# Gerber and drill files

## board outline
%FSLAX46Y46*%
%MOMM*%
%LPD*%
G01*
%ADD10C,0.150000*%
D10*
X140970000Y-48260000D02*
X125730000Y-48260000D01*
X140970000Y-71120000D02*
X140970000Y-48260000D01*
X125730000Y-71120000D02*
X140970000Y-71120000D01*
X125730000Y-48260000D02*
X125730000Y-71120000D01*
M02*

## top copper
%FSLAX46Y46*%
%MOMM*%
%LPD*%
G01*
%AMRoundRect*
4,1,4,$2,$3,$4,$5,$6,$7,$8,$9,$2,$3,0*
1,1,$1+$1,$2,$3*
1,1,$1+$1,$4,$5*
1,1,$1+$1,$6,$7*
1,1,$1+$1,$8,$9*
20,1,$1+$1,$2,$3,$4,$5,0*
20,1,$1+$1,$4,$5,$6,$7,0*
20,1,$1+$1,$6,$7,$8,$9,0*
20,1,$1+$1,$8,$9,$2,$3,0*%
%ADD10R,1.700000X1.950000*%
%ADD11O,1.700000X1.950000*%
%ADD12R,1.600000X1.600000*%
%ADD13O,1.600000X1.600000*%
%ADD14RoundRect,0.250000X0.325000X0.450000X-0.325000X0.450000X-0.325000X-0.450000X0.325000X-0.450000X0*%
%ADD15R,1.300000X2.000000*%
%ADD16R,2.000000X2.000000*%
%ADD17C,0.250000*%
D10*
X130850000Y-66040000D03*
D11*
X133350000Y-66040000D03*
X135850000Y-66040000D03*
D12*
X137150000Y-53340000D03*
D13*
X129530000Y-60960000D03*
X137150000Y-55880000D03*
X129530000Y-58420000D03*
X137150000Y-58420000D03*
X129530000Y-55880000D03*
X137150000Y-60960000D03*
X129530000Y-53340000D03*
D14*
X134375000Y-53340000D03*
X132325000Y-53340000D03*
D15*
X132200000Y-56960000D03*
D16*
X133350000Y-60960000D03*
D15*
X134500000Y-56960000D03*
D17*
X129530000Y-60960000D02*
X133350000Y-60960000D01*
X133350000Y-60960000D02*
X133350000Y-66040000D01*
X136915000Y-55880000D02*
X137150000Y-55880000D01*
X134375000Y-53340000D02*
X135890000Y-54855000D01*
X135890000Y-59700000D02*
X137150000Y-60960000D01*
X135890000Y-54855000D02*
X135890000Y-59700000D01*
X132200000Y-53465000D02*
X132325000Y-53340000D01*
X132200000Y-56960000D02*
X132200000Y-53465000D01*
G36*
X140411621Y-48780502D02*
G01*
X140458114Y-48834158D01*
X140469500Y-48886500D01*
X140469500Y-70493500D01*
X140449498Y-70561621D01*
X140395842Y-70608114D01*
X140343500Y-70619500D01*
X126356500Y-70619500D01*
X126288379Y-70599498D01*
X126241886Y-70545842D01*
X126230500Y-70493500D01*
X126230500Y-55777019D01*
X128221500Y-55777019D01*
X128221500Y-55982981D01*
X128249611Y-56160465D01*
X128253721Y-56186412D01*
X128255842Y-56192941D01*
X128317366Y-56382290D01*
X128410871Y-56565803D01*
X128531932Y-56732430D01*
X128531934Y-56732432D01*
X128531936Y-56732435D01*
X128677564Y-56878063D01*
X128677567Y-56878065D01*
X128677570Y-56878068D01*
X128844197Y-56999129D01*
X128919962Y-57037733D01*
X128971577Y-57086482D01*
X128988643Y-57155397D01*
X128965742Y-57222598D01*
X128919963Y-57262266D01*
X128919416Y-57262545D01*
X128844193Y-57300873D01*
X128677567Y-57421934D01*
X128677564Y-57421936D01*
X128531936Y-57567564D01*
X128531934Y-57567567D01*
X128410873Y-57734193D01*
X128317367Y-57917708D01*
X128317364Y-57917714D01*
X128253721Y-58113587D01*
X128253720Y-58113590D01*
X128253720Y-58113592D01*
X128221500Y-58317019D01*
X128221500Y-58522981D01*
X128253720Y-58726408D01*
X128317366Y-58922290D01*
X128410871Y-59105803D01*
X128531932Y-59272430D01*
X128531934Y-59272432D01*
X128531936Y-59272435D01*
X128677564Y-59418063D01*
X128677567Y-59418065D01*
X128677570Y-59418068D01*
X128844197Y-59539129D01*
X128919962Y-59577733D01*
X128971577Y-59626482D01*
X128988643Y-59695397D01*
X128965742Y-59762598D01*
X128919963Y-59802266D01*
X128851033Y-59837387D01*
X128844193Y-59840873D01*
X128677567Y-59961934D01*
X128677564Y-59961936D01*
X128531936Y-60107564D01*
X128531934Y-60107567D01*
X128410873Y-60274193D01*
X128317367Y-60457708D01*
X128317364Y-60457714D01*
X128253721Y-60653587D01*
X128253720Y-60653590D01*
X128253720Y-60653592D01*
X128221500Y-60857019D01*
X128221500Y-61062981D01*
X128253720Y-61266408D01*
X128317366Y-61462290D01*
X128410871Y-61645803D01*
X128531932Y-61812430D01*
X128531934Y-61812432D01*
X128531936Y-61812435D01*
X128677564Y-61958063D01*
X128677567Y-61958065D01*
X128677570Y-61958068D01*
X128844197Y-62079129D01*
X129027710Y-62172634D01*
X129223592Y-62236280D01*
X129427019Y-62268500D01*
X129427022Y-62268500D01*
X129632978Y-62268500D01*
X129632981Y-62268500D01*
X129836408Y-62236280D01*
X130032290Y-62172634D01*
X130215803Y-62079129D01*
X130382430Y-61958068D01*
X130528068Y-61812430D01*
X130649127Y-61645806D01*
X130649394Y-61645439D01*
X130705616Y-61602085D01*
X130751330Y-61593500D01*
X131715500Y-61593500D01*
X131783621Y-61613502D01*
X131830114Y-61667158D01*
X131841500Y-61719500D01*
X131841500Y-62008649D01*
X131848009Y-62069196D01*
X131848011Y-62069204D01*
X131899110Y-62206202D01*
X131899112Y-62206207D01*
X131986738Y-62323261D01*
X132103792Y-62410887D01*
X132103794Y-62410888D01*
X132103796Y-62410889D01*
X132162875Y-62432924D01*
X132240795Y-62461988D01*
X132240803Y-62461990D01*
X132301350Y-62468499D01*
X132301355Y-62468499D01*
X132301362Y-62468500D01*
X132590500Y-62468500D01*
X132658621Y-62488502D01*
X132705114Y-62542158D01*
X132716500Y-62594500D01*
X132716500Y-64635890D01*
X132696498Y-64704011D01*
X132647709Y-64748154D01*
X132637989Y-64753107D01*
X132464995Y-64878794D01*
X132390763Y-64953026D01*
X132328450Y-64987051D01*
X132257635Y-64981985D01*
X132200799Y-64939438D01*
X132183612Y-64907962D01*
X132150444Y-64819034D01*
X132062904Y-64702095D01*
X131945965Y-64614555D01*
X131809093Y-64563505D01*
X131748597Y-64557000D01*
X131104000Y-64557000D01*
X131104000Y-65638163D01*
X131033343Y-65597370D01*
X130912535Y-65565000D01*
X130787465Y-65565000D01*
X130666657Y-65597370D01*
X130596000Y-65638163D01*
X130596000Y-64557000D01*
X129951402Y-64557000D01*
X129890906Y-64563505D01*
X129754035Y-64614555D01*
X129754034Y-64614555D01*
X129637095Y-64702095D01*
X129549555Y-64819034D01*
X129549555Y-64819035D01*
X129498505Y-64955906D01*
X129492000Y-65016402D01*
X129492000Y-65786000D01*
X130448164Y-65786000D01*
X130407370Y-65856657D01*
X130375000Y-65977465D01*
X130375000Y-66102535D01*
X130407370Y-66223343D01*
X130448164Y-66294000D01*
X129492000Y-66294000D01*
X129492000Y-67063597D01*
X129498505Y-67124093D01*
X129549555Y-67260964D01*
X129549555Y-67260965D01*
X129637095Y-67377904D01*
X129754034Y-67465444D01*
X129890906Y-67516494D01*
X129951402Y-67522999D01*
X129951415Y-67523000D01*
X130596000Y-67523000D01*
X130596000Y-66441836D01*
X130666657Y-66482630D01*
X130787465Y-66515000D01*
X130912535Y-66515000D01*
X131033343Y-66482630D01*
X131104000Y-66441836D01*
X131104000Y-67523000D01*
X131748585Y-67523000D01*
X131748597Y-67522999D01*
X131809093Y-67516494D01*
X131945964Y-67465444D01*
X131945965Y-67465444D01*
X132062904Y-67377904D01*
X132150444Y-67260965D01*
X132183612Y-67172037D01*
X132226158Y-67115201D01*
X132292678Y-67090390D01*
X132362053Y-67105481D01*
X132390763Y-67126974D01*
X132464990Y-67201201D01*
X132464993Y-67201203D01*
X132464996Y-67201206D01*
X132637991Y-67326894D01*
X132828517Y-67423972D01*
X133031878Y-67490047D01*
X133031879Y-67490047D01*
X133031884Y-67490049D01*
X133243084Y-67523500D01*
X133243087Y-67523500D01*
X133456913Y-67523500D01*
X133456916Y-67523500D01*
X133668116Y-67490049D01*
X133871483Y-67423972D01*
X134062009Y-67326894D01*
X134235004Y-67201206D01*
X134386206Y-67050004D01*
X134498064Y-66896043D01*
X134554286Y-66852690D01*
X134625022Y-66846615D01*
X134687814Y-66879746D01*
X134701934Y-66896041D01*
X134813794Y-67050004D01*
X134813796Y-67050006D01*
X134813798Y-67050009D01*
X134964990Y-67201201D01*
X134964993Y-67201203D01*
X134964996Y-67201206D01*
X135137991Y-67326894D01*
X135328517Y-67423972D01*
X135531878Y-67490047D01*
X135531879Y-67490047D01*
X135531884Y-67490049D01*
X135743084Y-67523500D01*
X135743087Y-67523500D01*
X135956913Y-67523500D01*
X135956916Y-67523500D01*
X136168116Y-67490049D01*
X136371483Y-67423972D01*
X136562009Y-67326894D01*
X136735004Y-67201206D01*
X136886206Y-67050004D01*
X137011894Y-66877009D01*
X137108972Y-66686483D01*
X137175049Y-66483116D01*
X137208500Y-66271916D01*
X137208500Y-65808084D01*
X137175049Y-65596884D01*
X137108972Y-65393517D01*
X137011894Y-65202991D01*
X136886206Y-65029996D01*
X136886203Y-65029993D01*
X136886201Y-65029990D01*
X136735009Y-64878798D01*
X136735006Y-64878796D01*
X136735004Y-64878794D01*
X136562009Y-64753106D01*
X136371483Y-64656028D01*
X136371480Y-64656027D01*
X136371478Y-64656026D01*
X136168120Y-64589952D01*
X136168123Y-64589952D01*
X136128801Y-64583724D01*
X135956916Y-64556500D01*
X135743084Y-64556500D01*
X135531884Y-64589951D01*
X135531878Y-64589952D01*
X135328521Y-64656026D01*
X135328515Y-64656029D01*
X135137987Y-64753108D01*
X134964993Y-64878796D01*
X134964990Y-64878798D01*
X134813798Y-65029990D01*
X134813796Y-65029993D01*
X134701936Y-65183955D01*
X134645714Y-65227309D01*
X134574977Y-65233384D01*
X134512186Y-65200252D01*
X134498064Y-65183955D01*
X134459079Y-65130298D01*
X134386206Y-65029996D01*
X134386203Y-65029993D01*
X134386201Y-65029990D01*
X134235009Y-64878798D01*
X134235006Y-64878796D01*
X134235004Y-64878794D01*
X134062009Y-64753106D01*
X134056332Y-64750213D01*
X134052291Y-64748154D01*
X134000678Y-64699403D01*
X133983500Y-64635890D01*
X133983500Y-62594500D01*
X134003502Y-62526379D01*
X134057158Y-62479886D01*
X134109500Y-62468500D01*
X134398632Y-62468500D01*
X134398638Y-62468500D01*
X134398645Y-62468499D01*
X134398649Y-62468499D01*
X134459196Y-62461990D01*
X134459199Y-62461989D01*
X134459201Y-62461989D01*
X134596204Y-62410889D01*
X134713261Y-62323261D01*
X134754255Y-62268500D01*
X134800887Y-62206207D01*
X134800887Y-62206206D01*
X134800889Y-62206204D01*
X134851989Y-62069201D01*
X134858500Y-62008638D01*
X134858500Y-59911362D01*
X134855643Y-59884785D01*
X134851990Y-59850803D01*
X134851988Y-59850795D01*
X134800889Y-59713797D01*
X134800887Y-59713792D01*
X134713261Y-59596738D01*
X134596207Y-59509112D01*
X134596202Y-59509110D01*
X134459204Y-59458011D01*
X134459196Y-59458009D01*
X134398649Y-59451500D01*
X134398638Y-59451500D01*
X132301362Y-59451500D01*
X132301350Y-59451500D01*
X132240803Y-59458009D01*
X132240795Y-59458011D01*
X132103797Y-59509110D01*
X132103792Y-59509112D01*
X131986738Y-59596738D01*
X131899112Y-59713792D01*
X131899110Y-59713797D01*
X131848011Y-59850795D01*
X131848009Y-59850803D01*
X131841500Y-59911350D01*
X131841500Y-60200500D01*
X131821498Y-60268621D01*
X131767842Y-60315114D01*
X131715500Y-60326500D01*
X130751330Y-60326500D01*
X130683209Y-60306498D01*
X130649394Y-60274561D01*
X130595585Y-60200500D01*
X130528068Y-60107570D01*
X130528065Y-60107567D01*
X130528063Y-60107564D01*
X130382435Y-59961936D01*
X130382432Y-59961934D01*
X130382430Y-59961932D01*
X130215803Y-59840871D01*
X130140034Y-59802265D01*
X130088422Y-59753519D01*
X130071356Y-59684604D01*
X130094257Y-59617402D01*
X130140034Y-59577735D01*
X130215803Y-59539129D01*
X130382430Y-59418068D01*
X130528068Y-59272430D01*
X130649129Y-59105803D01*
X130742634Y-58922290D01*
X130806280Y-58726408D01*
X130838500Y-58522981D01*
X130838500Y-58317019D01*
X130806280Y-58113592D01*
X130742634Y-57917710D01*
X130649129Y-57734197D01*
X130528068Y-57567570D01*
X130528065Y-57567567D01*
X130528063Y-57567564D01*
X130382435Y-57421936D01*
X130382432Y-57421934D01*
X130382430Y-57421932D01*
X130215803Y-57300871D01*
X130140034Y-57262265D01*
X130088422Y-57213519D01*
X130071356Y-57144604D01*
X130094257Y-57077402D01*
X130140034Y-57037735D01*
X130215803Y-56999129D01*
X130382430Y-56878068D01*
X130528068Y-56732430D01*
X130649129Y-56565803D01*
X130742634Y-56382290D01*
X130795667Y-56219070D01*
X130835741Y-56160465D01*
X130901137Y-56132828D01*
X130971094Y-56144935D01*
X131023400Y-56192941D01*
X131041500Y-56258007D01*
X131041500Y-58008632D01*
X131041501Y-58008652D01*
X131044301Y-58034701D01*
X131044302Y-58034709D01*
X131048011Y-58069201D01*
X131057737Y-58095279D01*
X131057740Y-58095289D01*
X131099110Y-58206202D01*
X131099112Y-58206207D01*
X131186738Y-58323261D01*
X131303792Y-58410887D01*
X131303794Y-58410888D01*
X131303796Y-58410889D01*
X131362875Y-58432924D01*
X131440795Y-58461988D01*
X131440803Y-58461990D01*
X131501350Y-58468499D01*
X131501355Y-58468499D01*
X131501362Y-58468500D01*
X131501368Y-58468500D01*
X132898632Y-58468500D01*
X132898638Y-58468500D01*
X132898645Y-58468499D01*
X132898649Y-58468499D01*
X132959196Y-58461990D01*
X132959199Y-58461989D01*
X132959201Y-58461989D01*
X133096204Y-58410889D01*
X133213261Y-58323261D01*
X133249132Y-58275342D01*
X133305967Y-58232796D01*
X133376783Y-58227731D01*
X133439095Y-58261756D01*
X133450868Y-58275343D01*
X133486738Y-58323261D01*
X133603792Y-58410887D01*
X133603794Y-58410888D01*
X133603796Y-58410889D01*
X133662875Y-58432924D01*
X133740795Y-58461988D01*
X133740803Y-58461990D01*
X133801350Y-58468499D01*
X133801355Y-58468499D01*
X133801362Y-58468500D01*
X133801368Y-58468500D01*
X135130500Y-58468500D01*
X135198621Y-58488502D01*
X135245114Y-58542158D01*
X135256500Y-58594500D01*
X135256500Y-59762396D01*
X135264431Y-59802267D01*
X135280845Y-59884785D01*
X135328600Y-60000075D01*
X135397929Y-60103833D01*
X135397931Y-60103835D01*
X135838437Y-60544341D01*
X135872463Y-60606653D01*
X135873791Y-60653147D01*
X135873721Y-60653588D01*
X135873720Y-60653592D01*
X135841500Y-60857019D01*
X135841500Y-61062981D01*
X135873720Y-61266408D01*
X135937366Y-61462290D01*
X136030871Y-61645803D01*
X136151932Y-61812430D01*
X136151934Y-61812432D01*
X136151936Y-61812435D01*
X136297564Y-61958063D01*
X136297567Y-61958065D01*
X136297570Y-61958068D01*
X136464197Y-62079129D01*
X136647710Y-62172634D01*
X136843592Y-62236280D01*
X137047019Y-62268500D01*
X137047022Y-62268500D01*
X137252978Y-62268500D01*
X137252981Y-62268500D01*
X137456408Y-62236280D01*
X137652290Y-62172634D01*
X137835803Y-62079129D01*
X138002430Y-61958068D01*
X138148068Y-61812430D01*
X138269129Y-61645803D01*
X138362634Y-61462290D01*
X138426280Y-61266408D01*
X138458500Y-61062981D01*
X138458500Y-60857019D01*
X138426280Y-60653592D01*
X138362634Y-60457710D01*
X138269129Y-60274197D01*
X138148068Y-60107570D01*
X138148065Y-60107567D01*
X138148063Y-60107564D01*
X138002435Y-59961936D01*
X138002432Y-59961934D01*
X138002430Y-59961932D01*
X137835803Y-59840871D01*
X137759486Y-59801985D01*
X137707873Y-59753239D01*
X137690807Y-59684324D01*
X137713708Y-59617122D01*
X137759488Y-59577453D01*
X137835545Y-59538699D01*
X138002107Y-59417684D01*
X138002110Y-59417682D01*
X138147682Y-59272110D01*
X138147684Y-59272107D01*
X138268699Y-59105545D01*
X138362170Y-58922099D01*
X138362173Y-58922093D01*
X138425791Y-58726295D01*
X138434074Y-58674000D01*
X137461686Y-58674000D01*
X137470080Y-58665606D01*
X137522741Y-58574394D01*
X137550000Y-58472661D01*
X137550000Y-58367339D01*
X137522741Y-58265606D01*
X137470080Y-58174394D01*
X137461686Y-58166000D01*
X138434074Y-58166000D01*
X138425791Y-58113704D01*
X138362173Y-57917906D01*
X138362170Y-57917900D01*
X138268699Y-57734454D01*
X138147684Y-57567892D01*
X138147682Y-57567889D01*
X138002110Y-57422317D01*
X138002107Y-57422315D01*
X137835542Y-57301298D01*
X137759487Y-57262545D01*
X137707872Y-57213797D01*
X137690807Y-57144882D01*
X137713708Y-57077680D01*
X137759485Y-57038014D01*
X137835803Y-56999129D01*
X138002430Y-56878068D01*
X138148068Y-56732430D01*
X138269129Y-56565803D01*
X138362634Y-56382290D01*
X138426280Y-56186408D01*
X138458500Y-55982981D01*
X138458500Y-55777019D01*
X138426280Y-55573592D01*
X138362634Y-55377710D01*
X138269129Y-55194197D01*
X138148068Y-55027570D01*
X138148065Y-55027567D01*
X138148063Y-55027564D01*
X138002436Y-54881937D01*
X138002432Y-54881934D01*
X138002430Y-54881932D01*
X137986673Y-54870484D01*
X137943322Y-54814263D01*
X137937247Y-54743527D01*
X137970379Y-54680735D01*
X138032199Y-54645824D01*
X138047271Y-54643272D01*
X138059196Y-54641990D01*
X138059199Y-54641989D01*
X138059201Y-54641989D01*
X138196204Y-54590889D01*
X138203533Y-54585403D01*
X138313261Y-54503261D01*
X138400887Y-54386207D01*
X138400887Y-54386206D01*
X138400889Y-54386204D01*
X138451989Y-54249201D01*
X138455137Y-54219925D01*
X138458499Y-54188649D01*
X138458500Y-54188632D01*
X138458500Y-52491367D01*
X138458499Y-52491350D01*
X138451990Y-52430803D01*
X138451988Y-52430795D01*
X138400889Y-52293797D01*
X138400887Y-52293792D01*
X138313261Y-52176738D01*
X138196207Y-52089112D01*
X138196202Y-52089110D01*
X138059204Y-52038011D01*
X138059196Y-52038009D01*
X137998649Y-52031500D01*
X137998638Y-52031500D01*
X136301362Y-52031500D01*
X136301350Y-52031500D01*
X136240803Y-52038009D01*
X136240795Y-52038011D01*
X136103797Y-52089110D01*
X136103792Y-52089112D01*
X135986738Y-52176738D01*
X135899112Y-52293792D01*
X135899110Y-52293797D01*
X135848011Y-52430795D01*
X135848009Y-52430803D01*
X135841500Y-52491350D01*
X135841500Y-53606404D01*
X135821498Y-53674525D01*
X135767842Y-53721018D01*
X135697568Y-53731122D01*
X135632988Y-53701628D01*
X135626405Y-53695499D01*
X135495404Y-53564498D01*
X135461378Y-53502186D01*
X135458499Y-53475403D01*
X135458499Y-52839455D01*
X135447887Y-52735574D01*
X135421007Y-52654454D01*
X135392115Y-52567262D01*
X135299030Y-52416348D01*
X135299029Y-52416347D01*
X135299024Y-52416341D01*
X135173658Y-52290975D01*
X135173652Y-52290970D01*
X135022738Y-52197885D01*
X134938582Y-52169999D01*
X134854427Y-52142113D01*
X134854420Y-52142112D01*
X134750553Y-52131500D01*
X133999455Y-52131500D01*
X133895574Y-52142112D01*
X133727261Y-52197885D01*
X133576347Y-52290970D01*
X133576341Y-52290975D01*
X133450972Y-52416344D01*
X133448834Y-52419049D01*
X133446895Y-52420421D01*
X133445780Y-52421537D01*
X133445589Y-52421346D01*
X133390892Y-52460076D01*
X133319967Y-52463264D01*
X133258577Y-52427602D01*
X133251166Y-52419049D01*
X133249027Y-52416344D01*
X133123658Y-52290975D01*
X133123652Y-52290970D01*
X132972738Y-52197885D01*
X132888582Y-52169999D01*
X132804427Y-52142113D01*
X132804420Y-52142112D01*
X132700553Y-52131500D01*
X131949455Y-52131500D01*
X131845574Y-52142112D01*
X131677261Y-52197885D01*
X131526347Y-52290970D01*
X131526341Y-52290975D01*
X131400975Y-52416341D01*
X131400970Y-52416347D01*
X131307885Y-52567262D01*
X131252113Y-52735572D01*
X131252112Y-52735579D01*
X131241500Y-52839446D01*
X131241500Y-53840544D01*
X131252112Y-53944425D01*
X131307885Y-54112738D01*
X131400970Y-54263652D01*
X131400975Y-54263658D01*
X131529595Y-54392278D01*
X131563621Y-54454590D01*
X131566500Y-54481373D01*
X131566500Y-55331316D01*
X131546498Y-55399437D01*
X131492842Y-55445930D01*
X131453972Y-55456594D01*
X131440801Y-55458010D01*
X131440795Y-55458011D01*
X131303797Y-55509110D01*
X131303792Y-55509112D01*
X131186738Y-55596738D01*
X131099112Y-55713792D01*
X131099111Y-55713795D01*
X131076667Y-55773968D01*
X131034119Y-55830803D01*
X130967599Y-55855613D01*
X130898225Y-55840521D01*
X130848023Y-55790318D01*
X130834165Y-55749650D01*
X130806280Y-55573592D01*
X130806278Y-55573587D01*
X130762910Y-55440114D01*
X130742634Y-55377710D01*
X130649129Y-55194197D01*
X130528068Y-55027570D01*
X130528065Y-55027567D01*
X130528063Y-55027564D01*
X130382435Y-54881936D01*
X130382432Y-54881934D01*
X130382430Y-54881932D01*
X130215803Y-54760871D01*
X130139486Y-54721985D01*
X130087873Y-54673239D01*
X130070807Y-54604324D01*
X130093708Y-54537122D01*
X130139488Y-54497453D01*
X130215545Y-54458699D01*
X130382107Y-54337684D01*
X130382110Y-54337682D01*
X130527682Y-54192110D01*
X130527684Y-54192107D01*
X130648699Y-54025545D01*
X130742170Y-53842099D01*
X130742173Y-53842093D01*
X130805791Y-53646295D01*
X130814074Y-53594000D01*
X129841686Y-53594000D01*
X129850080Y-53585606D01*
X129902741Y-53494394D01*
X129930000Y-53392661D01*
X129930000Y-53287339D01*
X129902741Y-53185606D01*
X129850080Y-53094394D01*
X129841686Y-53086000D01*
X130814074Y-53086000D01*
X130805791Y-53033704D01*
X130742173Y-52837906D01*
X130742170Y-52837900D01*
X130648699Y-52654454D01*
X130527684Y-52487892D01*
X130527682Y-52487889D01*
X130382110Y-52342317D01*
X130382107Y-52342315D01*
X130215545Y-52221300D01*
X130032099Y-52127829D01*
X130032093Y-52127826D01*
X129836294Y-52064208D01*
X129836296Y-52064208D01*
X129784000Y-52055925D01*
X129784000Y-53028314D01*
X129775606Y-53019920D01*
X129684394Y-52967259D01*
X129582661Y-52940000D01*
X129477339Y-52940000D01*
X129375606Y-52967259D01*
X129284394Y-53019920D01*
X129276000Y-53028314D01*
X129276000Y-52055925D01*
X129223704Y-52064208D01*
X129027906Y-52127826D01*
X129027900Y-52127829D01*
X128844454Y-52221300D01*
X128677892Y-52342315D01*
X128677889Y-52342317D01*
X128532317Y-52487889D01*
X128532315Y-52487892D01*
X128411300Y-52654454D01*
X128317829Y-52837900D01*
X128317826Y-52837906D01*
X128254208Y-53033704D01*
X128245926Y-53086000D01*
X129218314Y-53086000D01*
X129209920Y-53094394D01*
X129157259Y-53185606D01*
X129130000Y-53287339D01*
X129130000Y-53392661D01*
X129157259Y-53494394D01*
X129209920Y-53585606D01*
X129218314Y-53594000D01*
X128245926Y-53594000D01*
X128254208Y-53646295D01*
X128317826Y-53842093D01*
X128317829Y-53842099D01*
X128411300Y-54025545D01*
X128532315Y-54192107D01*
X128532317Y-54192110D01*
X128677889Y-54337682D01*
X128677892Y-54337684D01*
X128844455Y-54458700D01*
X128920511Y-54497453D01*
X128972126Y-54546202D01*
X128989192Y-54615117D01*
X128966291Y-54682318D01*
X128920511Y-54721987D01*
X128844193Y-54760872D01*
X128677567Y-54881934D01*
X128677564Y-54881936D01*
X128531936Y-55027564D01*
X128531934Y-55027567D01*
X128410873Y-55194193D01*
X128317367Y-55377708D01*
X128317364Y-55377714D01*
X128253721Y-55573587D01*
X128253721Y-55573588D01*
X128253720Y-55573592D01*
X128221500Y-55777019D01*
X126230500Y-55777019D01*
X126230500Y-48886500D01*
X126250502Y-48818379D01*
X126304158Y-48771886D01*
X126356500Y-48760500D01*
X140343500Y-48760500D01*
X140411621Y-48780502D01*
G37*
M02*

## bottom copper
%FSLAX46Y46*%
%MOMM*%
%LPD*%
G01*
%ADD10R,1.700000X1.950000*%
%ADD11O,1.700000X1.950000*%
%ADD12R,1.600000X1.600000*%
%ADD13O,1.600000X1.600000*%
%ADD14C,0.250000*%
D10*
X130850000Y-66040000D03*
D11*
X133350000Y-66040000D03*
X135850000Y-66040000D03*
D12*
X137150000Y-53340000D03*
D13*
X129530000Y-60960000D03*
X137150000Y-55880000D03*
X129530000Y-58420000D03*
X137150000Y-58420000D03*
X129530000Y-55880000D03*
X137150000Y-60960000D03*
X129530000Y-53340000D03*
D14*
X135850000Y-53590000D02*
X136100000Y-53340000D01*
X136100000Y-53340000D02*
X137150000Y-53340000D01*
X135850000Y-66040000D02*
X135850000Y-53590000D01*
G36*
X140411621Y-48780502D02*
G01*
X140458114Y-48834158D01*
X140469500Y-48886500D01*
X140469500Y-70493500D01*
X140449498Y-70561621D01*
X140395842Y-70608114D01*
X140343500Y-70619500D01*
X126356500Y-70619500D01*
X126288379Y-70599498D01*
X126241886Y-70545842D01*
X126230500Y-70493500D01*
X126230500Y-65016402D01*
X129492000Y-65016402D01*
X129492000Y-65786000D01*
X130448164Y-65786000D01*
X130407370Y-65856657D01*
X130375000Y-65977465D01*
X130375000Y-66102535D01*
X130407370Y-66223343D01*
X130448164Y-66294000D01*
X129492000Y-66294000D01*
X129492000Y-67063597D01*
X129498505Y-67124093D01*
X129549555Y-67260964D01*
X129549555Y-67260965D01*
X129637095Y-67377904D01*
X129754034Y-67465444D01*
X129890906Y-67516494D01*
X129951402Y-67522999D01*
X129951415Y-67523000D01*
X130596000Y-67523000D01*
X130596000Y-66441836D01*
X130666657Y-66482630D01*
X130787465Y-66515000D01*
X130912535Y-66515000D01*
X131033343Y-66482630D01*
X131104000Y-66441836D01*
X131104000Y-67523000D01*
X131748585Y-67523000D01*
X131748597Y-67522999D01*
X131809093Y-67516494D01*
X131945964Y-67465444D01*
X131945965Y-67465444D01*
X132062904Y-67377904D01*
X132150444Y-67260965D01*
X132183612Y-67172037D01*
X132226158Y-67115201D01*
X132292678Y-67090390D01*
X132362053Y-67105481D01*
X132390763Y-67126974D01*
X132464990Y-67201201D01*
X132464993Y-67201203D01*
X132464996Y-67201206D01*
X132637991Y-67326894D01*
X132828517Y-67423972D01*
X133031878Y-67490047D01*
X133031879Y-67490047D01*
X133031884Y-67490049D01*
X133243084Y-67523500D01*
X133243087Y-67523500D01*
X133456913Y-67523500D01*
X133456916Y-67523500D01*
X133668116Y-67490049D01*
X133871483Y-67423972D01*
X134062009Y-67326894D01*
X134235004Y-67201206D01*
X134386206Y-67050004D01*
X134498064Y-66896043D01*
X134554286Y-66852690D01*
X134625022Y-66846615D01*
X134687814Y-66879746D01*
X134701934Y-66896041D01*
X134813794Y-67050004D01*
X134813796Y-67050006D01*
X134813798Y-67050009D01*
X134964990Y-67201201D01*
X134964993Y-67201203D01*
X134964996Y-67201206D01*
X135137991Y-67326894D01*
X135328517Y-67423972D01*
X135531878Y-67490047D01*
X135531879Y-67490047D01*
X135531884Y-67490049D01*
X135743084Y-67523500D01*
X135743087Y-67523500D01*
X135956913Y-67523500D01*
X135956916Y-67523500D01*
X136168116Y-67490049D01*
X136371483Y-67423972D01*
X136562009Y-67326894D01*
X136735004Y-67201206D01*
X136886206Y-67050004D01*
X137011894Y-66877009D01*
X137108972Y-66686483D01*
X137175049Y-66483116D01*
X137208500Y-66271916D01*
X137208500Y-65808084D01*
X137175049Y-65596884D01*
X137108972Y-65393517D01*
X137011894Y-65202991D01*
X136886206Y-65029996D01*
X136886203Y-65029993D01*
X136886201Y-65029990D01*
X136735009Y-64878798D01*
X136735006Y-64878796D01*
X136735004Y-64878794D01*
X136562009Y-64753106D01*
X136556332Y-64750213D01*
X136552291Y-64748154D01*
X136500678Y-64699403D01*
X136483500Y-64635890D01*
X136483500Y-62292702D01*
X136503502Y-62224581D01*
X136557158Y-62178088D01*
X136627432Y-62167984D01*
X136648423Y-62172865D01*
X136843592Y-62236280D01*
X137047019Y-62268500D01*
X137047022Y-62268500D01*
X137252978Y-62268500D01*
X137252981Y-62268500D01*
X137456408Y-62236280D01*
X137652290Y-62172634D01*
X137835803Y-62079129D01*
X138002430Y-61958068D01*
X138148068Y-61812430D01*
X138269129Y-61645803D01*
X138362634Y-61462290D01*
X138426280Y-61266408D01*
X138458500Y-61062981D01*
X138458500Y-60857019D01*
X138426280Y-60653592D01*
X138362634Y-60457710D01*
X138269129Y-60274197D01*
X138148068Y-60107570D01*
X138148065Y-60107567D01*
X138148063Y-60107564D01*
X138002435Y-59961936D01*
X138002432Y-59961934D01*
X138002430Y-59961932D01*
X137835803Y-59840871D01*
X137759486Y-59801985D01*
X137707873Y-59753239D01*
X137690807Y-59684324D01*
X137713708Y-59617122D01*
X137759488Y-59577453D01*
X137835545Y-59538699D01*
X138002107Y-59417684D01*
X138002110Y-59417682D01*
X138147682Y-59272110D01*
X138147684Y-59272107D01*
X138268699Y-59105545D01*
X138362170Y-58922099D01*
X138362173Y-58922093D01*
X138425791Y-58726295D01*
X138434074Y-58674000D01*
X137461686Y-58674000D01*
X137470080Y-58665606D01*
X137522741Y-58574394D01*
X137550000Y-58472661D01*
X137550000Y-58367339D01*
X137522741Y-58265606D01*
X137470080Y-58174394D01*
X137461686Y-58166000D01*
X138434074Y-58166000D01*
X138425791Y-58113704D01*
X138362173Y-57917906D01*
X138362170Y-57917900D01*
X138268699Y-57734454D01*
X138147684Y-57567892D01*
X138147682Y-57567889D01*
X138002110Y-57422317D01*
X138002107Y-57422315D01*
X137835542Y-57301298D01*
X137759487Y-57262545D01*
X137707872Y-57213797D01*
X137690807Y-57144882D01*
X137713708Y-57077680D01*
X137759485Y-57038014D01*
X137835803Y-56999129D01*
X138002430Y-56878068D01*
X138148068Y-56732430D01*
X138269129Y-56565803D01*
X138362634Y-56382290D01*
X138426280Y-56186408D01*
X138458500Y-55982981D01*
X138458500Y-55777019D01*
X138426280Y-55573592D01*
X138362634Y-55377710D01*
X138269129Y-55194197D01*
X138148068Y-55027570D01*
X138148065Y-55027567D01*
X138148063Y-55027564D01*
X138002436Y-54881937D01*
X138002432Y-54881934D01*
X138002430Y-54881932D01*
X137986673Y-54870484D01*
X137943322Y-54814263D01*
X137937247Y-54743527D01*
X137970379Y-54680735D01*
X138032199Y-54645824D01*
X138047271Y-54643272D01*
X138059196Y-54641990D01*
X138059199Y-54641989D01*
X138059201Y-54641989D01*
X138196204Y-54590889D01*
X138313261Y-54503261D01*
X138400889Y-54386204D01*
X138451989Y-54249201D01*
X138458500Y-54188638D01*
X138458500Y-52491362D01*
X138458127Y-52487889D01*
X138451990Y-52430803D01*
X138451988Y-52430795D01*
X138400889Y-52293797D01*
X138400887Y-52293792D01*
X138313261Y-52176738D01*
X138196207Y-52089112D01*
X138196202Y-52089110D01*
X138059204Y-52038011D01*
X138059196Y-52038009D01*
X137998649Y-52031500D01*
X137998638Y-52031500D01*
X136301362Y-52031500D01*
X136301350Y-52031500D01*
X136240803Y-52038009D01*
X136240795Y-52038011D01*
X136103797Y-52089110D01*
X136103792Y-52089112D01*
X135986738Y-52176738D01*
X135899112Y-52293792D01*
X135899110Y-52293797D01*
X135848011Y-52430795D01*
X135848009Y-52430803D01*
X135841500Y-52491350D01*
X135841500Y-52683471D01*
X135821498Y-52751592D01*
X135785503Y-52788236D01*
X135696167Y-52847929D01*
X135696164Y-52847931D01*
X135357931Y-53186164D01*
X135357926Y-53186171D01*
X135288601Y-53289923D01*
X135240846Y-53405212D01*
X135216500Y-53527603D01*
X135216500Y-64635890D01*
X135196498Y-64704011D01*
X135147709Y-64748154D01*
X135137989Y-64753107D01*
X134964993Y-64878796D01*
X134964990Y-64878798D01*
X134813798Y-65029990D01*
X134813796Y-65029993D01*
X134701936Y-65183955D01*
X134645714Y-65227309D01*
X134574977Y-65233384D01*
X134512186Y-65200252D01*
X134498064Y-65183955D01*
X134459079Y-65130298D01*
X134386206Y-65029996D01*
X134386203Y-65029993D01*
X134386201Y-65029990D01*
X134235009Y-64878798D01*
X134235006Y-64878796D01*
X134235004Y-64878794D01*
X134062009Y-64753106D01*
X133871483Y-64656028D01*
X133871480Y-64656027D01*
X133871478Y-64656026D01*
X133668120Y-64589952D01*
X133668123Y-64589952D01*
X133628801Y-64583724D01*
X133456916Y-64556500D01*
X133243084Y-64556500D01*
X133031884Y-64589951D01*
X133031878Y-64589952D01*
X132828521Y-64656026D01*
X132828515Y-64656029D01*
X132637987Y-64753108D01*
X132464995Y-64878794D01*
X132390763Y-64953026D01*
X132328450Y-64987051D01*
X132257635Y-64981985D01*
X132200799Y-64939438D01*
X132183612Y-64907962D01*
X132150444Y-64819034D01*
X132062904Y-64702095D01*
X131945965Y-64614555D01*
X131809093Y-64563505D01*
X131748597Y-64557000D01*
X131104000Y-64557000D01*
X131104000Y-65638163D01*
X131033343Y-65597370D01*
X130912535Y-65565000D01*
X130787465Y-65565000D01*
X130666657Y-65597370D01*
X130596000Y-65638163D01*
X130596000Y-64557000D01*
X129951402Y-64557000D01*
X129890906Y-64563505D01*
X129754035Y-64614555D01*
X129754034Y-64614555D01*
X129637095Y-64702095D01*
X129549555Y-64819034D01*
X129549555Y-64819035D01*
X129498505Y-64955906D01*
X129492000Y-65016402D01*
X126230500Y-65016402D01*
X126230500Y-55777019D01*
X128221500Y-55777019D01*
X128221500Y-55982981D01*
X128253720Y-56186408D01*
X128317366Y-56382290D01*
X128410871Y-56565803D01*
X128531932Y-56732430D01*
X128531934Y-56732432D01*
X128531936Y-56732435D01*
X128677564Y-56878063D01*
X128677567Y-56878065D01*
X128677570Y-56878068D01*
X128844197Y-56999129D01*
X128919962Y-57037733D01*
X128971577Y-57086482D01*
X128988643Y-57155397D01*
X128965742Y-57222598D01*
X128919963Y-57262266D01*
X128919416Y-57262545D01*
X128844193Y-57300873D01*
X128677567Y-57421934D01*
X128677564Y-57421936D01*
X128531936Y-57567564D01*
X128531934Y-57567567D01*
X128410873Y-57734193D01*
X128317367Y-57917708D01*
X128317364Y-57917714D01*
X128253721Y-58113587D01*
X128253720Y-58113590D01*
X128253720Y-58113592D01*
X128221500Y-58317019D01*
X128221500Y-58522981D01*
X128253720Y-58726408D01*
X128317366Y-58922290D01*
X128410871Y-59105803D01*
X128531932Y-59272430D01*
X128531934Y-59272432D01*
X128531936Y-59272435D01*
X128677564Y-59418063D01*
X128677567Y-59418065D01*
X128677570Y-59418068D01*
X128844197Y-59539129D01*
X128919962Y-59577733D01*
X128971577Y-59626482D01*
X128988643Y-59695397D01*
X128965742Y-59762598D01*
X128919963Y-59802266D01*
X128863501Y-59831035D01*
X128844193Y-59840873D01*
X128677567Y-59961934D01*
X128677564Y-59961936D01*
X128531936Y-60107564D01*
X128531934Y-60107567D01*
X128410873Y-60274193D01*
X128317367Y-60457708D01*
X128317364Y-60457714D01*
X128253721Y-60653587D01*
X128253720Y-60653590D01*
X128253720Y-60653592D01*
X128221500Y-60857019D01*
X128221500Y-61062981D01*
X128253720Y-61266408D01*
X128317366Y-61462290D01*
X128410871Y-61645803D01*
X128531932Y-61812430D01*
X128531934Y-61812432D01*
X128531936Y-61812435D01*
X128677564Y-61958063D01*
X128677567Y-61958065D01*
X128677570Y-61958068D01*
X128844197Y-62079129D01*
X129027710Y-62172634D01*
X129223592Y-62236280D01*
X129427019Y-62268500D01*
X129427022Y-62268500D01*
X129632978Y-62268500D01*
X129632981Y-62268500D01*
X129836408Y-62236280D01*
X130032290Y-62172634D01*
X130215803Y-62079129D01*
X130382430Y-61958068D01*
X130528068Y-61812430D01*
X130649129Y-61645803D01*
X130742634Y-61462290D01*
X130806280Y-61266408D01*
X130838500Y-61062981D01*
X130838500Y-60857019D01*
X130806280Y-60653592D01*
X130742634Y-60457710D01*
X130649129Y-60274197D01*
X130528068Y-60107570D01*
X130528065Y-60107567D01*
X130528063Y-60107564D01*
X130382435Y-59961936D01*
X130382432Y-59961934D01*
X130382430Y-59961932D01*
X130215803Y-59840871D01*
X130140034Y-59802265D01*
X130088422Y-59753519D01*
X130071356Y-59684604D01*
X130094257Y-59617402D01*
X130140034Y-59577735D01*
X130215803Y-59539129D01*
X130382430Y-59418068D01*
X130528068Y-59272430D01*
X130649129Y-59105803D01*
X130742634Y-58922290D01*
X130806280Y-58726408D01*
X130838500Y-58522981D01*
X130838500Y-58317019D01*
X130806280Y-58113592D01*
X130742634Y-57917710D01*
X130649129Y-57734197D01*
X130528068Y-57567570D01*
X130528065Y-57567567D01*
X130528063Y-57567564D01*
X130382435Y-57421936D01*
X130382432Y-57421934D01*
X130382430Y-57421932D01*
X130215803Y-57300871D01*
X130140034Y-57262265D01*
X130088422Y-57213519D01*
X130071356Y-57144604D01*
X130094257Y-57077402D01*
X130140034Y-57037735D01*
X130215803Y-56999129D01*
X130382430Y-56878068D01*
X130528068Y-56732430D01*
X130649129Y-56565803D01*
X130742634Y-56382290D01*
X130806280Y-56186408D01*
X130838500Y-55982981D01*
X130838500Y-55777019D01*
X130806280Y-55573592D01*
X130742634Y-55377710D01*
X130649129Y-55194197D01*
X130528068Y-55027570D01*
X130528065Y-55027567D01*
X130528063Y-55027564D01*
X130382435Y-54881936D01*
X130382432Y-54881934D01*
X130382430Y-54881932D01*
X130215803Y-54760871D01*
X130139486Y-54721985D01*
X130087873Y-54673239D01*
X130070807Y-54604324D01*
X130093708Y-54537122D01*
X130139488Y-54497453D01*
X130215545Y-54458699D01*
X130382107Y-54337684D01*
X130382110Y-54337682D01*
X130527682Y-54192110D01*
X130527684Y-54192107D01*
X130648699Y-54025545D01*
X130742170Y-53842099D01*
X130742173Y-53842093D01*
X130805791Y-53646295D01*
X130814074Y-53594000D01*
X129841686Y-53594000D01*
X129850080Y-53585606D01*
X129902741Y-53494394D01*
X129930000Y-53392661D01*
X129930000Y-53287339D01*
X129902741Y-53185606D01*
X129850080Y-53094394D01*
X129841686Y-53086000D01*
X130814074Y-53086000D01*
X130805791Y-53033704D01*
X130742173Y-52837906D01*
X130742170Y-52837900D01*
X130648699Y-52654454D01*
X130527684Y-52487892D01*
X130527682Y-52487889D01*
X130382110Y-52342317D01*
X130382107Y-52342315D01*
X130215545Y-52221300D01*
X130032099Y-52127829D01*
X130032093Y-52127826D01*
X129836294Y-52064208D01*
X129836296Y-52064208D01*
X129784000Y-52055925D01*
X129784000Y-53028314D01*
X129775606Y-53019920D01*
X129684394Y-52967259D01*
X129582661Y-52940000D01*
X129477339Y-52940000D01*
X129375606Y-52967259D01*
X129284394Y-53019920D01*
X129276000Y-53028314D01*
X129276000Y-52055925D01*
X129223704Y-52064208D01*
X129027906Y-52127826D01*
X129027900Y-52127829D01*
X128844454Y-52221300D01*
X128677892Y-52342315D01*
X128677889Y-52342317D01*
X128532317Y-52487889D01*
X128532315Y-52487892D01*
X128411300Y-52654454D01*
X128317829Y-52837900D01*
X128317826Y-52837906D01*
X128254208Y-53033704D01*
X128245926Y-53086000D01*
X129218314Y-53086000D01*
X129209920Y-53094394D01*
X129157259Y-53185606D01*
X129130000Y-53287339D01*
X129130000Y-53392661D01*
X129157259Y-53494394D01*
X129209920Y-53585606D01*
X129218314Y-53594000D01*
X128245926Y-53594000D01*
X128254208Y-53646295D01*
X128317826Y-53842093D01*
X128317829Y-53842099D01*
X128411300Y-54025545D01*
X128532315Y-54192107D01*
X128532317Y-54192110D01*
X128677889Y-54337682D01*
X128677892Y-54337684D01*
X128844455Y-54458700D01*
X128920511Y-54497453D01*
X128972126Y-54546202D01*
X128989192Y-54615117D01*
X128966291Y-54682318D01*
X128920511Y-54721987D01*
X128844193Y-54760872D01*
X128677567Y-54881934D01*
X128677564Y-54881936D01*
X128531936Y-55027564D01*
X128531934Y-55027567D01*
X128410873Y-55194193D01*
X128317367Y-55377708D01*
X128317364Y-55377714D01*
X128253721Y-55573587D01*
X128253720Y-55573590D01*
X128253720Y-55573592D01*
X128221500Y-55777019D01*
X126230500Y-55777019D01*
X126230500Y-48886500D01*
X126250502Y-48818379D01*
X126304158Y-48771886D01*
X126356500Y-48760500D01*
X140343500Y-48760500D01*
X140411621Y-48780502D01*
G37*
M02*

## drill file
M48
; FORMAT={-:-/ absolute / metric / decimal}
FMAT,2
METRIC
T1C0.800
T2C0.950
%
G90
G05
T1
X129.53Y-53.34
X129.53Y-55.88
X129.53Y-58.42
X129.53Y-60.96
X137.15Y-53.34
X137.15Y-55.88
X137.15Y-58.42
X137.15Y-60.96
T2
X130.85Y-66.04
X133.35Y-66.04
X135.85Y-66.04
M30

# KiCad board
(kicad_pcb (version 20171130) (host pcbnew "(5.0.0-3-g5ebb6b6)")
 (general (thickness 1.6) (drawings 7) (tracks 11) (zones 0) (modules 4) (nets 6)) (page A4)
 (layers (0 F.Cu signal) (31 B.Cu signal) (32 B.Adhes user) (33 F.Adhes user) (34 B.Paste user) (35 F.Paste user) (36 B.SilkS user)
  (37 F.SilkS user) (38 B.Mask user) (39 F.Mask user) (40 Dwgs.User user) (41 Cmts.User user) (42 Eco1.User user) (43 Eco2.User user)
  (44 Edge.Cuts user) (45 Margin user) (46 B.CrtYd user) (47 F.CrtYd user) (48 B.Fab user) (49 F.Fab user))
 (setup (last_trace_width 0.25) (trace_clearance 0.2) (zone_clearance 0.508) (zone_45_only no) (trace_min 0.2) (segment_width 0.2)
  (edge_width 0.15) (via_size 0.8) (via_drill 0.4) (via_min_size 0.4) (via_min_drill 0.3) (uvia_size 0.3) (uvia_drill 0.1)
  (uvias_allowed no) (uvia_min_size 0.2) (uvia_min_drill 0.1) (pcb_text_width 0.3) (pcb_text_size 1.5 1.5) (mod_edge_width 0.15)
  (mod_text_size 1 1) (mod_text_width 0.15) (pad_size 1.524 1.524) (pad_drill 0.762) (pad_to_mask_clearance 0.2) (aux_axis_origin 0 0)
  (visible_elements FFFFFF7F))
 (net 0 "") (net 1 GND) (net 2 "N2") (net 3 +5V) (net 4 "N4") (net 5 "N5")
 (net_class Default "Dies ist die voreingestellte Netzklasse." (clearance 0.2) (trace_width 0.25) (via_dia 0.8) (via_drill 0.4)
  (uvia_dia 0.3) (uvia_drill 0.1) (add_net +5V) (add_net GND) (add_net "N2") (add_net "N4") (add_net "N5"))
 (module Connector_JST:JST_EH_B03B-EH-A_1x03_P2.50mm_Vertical (layer F.Cu) (at 130.85 66.04)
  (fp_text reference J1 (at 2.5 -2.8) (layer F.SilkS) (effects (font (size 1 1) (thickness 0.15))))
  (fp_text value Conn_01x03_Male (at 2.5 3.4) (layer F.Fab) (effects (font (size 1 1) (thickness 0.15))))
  (pad 1 thru_hole rect (at 0 0) (size 1.7 1.95) (drill 0.95) (layers *.Cu *.Mask) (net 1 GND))
  (pad 2 thru_hole oval (at 2.5 0) (size 1.7 1.95) (drill 0.95) (layers *.Cu *.Mask) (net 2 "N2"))
  (pad 3 thru_hole oval (at 5 0) (size 1.7 1.95) (drill 0.95) (layers *.Cu *.Mask) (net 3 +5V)))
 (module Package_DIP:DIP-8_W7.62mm (layer B.Cu) (at 137.15 53.34 180)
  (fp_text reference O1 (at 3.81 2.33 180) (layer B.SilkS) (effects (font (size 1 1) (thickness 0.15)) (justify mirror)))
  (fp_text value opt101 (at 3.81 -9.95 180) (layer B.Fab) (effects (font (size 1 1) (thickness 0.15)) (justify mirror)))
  (pad 1 thru_hole rect (at 0 0 180) (size 1.6 1.6) (drill 0.8) (layers *.Cu *.Mask) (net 3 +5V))
  (pad 5 thru_hole oval (at 7.62 -7.62 180) (size 1.6 1.6) (drill 0.8) (layers *.Cu *.Mask) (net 2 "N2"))
  (pad 2 thru_hole oval (at 0 -2.54 180) (size 1.6 1.6) (drill 0.8) (layers *.Cu *.Mask))
  (pad 6 thru_hole oval (at 7.62 -5.08 180) (size 1.6 1.6) (drill 0.8) (layers *.Cu *.Mask))
  (pad 3 thru_hole oval (at 0 -5.08 180) (size 1.6 1.6) (drill 0.8) (layers *.Cu *.Mask) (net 1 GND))
  (pad 7 thru_hole oval (at 7.62 -2.54 180) (size 1.6 1.6) (drill 0.8) (layers *.Cu *.Mask))
  (pad 4 thru_hole oval (at 0 -7.62 180) (size 1.6 1.6) (drill 0.8) (layers *.Cu *.Mask) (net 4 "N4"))
  (pad 8 thru_hole oval (at 7.62 0 180) (size 1.6 1.6) (drill 0.8) (layers *.Cu *.Mask) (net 1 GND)))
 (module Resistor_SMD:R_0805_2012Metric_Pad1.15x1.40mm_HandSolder (layer F.Cu) (at 133.35 53.34 180)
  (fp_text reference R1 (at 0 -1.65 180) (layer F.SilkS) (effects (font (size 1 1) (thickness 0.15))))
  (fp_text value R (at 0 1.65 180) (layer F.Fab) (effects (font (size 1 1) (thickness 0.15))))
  (pad 1 smd roundrect (at -1.025 0 180) (size 1.15 1.4) (layers F.Cu F.Paste F.Mask) (roundrect_rratio 0.217391) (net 4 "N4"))
  (pad 2 smd roundrect (at 1.025 0 180) (size 1.15 1.4) (layers F.Cu F.Paste F.Mask) (roundrect_rratio 0.217391) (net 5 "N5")))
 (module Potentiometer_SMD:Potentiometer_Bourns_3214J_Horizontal (layer F.Cu) (at 133.35 58.96 90)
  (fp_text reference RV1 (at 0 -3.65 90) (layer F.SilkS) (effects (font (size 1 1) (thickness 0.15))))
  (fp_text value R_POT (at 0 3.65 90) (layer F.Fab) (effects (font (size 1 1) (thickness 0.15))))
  (pad 1 smd rect (at 2 -1.15 90) (size 2 1.3) (layers F.Cu F.Paste F.Mask) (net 5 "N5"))
  (pad 2 smd rect (at -2 0 90) (size 2 2) (layers F.Cu F.Paste F.Mask) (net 2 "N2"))
  (pad 3 smd rect (at 2 1.15 90) (size 2 1.3) (layers F.Cu F.Paste F.Mask)))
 (gr_line (start 140.97 48.26) (end 125.73 48.26) (layer Edge.Cuts) (width 0.15))
 (gr_line (start 140.97 71.12) (end 140.97 48.26) (layer Edge.Cuts) (width 0.15))
 (gr_line (start 125.73 71.12) (end 140.97 71.12) (layer Edge.Cuts) (width 0.15))
 (gr_line (start 125.73 48.26) (end 125.73 71.12) (layer Edge.Cuts) (width 0.15))
 (segment (start 129.53 60.96) (end 133.35 60.96) (width 0.25) (layer F.Cu) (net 2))
 (segment (start 133.35 60.96) (end 133.35 66.04) (width 0.25) (layer F.Cu) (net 2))
 (segment (start 135.85 53.59) (end 136.1 53.34) (width 0.25) (layer B.Cu) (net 3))
 (segment (start 136.1 53.34) (end 137.15 53.34) (width 0.25) (layer B.Cu) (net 3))
 (segment (start 135.85 66.04) (end 135.85 53.59) (width 0.25) (layer B.Cu) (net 3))
 (segment (start 136.915 55.88) (end 137.15 55.88) (width 0.25) (layer F.Cu) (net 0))
 (segment (start 134.375 53.34) (end 135.89 54.855) (width 0.25) (layer F.Cu) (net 4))
 (segment (start 135.89 59.7) (end 137.15 60.96) (width 0.25) (layer F.Cu) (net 4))
 (segment (start 135.89 54.855) (end 135.89 59.7) (width 0.25) (layer F.Cu) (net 4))
 (segment (start 132.2 53.465) (end 132.325 53.34) (width 0.25) (layer F.Cu) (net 5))
 (segment (start 132.2 56.96) (end 132.2 53.465) (width 0.25) (layer F.Cu) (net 5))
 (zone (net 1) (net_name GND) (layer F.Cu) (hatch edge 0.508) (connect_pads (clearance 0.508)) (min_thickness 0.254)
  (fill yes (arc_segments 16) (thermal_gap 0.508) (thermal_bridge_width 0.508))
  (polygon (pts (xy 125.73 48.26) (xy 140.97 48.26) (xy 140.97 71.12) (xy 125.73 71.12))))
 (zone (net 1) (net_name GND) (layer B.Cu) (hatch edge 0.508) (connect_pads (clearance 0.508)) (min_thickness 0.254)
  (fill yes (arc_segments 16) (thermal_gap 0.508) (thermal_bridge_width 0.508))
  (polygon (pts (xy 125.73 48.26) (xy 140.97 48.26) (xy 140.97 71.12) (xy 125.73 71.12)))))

